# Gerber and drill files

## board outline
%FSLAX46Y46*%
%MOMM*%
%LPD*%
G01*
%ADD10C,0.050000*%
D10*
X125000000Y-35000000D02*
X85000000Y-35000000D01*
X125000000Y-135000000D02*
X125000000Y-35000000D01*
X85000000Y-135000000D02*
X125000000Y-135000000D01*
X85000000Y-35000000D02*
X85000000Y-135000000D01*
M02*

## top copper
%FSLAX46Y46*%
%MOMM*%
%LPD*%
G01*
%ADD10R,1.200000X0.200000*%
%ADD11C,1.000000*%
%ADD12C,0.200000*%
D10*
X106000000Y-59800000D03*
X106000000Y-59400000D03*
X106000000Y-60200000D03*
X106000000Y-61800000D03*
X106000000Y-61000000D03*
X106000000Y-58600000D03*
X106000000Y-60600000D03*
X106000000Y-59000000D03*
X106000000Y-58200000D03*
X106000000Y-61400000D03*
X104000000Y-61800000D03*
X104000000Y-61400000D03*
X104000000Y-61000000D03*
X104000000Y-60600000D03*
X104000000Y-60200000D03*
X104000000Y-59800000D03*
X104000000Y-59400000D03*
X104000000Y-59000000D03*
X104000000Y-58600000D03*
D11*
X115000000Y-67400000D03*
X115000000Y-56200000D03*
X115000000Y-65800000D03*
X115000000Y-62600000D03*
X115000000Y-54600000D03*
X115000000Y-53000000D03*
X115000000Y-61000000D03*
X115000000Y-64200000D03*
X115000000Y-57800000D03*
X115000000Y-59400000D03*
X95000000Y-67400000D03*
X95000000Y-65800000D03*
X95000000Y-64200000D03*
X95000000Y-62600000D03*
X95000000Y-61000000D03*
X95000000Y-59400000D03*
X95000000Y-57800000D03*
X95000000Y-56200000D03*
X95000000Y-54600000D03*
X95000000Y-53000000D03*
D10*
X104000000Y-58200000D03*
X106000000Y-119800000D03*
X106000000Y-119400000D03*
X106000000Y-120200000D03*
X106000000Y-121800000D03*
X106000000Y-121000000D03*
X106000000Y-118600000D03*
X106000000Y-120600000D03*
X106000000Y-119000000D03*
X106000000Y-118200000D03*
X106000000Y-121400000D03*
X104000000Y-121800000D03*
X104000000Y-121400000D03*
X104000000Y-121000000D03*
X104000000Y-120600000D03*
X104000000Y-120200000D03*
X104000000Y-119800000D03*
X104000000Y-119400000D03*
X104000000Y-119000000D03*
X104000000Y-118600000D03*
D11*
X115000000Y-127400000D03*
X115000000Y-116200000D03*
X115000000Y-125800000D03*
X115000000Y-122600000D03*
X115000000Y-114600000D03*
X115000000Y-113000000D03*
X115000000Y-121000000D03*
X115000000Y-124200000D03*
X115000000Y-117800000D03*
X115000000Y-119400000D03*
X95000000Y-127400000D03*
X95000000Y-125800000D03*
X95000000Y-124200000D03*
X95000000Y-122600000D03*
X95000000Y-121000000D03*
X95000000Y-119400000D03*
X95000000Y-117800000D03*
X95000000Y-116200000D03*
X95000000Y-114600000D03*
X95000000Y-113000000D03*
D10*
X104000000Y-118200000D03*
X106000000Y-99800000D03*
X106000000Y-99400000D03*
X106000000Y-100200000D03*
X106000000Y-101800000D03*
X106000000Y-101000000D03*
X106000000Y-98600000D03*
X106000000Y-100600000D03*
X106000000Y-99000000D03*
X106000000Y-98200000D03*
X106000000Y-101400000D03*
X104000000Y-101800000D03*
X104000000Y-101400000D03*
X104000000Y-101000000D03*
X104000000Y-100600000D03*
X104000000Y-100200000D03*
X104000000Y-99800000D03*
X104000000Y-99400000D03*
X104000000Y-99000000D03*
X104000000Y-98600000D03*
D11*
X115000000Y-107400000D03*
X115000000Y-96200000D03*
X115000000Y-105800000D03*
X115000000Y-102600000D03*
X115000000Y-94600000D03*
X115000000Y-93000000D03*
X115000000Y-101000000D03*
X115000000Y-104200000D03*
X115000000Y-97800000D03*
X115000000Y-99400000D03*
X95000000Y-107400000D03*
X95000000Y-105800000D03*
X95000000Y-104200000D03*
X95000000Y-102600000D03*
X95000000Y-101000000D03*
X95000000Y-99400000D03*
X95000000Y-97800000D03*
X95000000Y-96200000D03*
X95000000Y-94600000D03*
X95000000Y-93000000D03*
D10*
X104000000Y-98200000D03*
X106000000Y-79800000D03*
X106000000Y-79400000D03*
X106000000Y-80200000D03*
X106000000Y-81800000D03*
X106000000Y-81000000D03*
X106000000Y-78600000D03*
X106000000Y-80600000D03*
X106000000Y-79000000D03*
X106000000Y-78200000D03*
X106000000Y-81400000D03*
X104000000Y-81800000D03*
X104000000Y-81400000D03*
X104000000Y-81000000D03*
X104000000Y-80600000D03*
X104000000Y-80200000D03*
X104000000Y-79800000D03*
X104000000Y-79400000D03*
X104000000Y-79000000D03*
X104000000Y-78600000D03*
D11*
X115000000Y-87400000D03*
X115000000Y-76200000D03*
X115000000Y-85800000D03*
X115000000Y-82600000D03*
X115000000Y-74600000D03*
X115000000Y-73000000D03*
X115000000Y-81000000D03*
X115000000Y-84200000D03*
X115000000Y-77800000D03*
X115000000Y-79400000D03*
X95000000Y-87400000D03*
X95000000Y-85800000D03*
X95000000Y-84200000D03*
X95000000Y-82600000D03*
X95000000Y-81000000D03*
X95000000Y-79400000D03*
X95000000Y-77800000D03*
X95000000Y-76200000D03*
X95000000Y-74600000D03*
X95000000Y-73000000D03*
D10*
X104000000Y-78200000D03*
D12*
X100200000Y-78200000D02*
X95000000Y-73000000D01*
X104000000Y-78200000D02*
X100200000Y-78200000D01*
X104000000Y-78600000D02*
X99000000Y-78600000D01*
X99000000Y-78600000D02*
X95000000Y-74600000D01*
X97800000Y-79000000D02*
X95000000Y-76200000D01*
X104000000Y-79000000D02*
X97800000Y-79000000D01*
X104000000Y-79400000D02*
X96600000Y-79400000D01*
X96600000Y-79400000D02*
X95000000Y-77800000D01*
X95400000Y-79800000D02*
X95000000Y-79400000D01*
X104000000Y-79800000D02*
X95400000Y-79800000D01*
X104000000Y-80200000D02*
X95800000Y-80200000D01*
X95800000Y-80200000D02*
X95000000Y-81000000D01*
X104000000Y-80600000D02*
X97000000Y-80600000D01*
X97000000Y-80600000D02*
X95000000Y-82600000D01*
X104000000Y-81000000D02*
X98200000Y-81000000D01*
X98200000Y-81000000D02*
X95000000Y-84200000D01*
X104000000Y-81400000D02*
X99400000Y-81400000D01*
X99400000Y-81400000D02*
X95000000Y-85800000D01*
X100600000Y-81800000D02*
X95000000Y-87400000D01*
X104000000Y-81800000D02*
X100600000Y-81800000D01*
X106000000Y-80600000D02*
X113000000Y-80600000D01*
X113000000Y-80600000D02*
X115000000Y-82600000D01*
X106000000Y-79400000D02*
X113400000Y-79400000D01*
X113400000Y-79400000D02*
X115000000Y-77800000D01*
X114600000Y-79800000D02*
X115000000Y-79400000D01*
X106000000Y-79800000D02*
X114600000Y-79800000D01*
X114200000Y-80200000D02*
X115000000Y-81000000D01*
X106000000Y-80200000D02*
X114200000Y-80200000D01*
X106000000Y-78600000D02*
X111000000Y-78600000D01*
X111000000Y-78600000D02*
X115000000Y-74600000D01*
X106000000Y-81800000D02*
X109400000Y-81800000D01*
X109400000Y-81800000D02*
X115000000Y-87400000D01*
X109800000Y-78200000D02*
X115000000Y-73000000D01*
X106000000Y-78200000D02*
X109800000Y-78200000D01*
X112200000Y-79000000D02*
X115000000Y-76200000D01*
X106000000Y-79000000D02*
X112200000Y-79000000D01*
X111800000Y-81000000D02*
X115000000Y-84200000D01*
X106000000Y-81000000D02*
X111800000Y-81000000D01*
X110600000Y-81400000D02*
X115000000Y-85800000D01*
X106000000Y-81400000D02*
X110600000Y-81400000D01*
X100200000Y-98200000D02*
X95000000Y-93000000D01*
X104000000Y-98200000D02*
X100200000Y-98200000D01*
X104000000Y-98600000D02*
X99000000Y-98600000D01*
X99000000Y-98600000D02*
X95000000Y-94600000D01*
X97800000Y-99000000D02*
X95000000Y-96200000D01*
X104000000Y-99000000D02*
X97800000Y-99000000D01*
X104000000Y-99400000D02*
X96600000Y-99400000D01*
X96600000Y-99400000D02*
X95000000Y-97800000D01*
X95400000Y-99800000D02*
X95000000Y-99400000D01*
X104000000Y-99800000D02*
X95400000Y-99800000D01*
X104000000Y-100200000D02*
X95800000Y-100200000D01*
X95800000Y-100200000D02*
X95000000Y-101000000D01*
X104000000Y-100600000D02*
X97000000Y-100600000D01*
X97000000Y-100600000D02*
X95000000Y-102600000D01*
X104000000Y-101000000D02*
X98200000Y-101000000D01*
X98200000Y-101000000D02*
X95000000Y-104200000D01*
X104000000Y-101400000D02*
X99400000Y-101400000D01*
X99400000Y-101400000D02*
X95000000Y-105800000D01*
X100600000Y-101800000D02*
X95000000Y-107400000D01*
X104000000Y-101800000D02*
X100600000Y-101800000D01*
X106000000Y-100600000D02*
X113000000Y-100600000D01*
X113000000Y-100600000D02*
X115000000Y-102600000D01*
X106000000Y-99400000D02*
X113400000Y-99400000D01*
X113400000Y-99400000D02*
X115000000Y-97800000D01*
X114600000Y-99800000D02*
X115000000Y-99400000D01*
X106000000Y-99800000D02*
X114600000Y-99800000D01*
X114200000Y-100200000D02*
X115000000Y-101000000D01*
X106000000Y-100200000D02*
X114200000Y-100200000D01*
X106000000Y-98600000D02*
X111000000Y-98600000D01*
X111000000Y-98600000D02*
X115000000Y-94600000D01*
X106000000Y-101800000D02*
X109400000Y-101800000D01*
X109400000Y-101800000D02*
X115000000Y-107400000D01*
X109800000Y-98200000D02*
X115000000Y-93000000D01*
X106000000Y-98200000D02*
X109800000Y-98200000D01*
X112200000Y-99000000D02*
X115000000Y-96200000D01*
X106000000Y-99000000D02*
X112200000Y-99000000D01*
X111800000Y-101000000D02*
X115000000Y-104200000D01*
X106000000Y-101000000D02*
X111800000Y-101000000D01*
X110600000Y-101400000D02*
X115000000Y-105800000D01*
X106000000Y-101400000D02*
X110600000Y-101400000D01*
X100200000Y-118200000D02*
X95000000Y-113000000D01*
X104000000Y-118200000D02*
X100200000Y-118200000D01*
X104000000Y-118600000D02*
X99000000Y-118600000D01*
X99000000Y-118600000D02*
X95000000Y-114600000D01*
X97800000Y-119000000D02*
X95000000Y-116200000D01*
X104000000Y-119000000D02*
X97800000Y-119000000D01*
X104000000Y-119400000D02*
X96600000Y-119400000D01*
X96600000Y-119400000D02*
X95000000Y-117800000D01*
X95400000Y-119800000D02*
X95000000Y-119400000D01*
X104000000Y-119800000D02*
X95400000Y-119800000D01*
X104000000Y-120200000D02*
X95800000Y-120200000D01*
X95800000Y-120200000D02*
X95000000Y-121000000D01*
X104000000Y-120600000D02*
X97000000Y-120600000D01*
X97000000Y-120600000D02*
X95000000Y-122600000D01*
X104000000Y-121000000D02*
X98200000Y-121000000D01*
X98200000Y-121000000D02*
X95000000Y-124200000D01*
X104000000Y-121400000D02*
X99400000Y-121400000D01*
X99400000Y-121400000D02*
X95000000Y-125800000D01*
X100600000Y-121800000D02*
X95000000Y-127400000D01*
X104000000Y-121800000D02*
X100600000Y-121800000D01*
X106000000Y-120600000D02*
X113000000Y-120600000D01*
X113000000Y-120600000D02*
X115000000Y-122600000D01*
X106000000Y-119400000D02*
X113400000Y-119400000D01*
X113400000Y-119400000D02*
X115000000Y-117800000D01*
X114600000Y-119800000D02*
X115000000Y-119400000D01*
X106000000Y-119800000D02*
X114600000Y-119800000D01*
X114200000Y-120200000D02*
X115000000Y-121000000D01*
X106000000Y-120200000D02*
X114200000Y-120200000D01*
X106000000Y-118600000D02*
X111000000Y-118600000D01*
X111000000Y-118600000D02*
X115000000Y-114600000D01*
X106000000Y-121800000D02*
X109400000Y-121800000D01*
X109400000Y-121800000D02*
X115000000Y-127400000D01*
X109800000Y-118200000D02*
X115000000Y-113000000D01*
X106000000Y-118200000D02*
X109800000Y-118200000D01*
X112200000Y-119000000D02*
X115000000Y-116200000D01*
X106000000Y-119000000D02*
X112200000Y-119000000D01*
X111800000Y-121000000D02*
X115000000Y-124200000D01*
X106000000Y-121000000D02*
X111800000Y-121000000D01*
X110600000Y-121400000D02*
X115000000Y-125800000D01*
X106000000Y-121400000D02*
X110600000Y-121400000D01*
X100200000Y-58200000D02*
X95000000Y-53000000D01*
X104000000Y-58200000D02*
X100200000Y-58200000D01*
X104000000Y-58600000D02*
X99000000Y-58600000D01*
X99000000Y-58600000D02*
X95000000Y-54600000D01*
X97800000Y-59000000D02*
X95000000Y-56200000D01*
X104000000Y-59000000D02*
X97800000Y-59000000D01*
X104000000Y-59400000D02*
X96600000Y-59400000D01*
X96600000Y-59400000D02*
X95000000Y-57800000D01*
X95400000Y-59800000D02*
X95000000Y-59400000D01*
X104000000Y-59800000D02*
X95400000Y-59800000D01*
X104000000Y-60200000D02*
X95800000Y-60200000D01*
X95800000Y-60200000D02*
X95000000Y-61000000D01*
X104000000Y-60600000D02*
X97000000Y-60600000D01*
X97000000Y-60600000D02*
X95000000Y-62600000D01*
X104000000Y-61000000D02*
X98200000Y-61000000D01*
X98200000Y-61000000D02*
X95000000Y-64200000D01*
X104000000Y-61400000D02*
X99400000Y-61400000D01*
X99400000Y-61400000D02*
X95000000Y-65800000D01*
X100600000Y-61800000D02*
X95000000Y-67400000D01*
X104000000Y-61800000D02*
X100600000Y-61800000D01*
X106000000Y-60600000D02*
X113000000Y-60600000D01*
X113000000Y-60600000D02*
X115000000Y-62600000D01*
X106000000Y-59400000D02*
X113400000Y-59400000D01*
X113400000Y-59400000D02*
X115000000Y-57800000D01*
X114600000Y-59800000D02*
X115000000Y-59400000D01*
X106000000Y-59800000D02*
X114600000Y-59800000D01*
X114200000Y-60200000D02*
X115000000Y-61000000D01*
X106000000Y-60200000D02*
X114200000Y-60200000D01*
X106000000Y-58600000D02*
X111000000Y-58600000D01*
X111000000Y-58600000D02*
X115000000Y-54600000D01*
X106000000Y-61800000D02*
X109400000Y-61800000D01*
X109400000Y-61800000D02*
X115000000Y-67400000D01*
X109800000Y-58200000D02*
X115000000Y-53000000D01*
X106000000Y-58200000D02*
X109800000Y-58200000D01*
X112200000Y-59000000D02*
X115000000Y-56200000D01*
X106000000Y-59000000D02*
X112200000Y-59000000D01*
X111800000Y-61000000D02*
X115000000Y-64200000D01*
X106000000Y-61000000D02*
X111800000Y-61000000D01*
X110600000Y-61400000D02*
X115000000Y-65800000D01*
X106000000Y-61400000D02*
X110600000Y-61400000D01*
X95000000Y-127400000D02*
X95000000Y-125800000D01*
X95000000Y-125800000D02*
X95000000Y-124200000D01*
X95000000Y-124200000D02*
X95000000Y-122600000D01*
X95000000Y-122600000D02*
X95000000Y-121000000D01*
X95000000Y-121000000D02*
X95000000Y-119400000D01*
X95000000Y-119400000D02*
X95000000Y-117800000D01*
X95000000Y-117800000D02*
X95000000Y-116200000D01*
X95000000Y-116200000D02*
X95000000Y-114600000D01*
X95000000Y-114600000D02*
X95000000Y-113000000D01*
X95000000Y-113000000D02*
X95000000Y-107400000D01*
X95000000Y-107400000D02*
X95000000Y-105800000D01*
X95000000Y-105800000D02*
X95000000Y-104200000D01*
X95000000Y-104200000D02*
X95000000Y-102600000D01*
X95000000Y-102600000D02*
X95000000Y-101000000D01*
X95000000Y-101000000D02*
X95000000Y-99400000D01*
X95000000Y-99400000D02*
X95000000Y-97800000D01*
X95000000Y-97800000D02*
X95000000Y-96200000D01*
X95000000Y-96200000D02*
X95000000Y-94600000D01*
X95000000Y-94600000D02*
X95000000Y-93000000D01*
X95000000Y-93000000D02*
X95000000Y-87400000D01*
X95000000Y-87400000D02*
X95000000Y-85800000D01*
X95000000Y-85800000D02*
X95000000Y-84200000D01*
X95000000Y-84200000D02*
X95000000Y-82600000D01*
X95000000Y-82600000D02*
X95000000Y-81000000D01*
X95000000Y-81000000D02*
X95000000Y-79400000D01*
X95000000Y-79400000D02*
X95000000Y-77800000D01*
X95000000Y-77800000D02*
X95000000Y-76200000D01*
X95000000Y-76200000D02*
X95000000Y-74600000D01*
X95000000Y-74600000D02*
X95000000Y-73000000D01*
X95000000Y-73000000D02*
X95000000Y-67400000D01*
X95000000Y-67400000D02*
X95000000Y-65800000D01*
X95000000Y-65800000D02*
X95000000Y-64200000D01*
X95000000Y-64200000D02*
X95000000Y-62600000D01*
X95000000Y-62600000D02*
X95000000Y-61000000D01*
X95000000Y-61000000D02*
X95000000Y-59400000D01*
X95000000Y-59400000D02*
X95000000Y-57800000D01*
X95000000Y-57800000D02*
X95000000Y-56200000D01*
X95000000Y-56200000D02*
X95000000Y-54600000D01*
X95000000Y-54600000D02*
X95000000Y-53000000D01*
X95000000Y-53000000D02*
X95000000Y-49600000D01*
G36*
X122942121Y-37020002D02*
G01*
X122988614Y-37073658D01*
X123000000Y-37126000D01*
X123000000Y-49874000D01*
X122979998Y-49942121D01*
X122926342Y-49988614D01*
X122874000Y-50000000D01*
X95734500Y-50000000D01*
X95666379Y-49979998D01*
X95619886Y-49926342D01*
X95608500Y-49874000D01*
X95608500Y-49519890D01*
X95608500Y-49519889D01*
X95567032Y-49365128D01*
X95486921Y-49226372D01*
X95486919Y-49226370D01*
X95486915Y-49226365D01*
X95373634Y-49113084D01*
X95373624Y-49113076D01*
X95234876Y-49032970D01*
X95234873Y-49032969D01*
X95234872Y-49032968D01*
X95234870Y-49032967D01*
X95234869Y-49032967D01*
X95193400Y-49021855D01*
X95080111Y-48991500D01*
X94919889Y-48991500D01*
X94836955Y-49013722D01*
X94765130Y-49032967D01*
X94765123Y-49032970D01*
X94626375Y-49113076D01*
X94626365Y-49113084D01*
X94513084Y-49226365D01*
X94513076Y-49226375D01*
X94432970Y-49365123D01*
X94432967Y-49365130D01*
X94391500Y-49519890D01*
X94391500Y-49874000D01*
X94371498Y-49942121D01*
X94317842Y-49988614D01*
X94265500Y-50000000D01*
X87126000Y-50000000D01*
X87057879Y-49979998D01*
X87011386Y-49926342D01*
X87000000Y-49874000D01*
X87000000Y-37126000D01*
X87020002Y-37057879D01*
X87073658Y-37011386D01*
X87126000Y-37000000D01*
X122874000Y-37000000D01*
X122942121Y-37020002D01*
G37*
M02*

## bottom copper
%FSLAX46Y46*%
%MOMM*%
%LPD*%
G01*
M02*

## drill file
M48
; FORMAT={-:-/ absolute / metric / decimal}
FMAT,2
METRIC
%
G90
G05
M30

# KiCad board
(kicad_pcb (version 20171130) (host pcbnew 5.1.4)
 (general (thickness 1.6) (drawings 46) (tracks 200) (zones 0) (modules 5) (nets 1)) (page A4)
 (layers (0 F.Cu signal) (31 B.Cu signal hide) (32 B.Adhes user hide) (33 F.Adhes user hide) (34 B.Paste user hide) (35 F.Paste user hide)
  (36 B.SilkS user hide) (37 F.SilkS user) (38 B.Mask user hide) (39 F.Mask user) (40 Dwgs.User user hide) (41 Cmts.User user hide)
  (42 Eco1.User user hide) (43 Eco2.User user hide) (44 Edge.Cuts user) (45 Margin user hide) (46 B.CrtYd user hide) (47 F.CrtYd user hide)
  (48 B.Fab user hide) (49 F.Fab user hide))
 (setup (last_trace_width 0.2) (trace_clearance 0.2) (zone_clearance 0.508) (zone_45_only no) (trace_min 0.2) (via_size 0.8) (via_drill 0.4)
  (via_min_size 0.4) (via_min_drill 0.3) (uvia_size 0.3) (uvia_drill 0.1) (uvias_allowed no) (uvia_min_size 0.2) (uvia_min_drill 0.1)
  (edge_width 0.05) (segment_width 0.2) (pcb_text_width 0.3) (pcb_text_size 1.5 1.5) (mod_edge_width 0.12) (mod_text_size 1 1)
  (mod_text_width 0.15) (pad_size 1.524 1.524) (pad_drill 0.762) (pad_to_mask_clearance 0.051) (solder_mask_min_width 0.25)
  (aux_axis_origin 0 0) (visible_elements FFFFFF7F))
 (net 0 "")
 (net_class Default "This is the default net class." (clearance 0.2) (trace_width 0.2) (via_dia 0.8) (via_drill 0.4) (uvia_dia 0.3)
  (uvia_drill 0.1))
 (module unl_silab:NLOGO (layer F.Cu) (at 87.6 132.2)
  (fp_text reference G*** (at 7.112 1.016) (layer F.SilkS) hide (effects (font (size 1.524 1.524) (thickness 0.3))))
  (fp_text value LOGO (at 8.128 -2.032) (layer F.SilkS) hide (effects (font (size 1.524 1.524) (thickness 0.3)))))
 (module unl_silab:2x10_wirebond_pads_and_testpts (layer F.Cu) (at 105 60)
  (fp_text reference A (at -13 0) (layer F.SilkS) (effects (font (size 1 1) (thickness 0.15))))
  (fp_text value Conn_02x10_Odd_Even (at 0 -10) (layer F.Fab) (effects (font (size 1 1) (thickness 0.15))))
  (pad 15 smd rect (at 1 -0.2) (size 1.2 0.2) (layers F.Cu F.Paste F.Mask))
  (pad 14 smd rect (at 1 -0.6) (size 1.2 0.2) (layers F.Cu F.Paste F.Mask))
  (pad 16 smd rect (at 1 0.2) (size 1.2 0.2) (layers F.Cu F.Paste F.Mask))
  (pad 20 smd rect (at 1 1.8) (size 1.2 0.2) (layers F.Cu F.Paste F.Mask))
  (pad 18 smd rect (at 1 1) (size 1.2 0.2) (layers F.Cu F.Paste F.Mask))
  (pad 12 smd rect (at 1 -1.4) (size 1.2 0.2) (layers F.Cu F.Paste F.Mask))
  (pad 17 smd rect (at 1 0.6) (size 1.2 0.2) (layers F.Cu F.Paste F.Mask))
  (pad 13 smd rect (at 1 -1) (size 1.2 0.2) (layers F.Cu F.Paste F.Mask))
  (pad 11 smd rect (at 1 -1.8) (size 1.2 0.2) (layers F.Cu F.Paste F.Mask))
  (pad 19 smd rect (at 1 1.4) (size 1.2 0.2) (layers F.Cu F.Paste F.Mask))
  (pad 10 smd rect (at -1 1.8) (size 1.2 0.2) (layers F.Cu F.Paste F.Mask))
  (pad 9 smd rect (at -1 1.4) (size 1.2 0.2) (layers F.Cu F.Paste F.Mask))
  (pad 8 smd rect (at -1 1) (size 1.2 0.2) (layers F.Cu F.Paste F.Mask))
  (pad 7 smd rect (at -1 0.6) (size 1.2 0.2) (layers F.Cu F.Paste F.Mask))
  (pad 6 smd rect (at -1 0.2) (size 1.2 0.2) (layers F.Cu F.Paste F.Mask))
  (pad 5 smd rect (at -1 -0.2) (size 1.2 0.2) (layers F.Cu F.Paste F.Mask))
  (pad 4 smd rect (at -1 -0.6) (size 1.2 0.2) (layers F.Cu F.Paste F.Mask))
  (pad 3 smd rect (at -1 -1) (size 1.2 0.2) (layers F.Cu F.Paste F.Mask))
  (pad 2 smd rect (at -1 -1.4) (size 1.2 0.2) (layers F.Cu F.Paste F.Mask))
  (pad 20 smd circle (at 10 7.4) (size 1 1) (layers F.Cu F.Paste F.Mask))
  (pad 13 smd circle (at 10 -3.8) (size 1 1) (layers F.Cu F.Paste F.Mask))
  (pad 19 smd circle (at 10 5.8) (size 1 1) (layers F.Cu F.Paste F.Mask))
  (pad 17 smd circle (at 10 2.6) (size 1 1) (layers F.Cu F.Paste F.Mask))
  (pad 12 smd circle (at 10 -5.4) (size 1 1) (layers F.Cu F.Paste F.Mask))
  (pad 11 smd circle (at 10 -7) (size 1 1) (layers F.Cu F.Paste F.Mask))
  (pad 16 smd circle (at 10 1) (size 1 1) (layers F.Cu F.Paste F.Mask))
  (pad 18 smd circle (at 10 4.2) (size 1 1) (layers F.Cu F.Paste F.Mask))
  (pad 14 smd circle (at 10 -2.2) (size 1 1) (layers F.Cu F.Paste F.Mask))
  (pad 15 smd circle (at 10 -0.6) (size 1 1) (layers F.Cu F.Paste F.Mask))
  (pad 10 smd circle (at -10 7.4) (size 1 1) (layers F.Cu F.Paste F.Mask))
  (pad 9 smd circle (at -10 5.8) (size 1 1) (layers F.Cu F.Paste F.Mask))
  (pad 8 smd circle (at -10 4.2) (size 1 1) (layers F.Cu F.Paste F.Mask))
  (pad 7 smd circle (at -10 2.6) (size 1 1) (layers F.Cu F.Paste F.Mask))
  (pad 6 smd circle (at -10 1) (size 1 1) (layers F.Cu F.Paste F.Mask))
  (pad 5 smd circle (at -10 -0.6) (size 1 1) (layers F.Cu F.Paste F.Mask))
  (pad 4 smd circle (at -10 -2.2) (size 1 1) (layers F.Cu F.Paste F.Mask))
  (pad 3 smd circle (at -10 -3.8) (size 1 1) (layers F.Cu F.Paste F.Mask))
  (pad 2 smd circle (at -10 -5.4) (size 1 1) (layers F.Cu F.Paste F.Mask))
  (pad 1 smd circle (at -10 -7) (size 1 1) (layers F.Cu F.Paste F.Mask))
  (pad 1 smd rect (at -1 -1.8) (size 1.2 0.2) (layers F.Cu F.Paste F.Mask)))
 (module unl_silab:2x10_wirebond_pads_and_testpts (layer F.Cu) (at 105 120)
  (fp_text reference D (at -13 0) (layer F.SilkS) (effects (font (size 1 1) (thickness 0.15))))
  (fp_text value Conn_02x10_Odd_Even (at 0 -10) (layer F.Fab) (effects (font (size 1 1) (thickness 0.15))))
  (pad 15 smd rect (at 1 -0.2) (size 1.2 0.2) (layers F.Cu F.Paste F.Mask))
  (pad 14 smd rect (at 1 -0.6) (size 1.2 0.2) (layers F.Cu F.Paste F.Mask))
  (pad 16 smd rect (at 1 0.2) (size 1.2 0.2) (layers F.Cu F.Paste F.Mask))
  (pad 20 smd rect (at 1 1.8) (size 1.2 0.2) (layers F.Cu F.Paste F.Mask))
  (pad 18 smd rect (at 1 1) (size 1.2 0.2) (layers F.Cu F.Paste F.Mask))
  (pad 12 smd rect (at 1 -1.4) (size 1.2 0.2) (layers F.Cu F.Paste F.Mask))
  (pad 17 smd rect (at 1 0.6) (size 1.2 0.2) (layers F.Cu F.Paste F.Mask))
  (pad 13 smd rect (at 1 -1) (size 1.2 0.2) (layers F.Cu F.Paste F.Mask))
  (pad 11 smd rect (at 1 -1.8) (size 1.2 0.2) (layers F.Cu F.Paste F.Mask))
  (pad 19 smd rect (at 1 1.4) (size 1.2 0.2) (layers F.Cu F.Paste F.Mask))
  (pad 10 smd rect (at -1 1.8) (size 1.2 0.2) (layers F.Cu F.Paste F.Mask))
  (pad 9 smd rect (at -1 1.4) (size 1.2 0.2) (layers F.Cu F.Paste F.Mask))
  (pad 8 smd rect (at -1 1) (size 1.2 0.2) (layers F.Cu F.Paste F.Mask))
  (pad 7 smd rect (at -1 0.6) (size 1.2 0.2) (layers F.Cu F.Paste F.Mask))
  (pad 6 smd rect (at -1 0.2) (size 1.2 0.2) (layers F.Cu F.Paste F.Mask))
  (pad 5 smd rect (at -1 -0.2) (size 1.2 0.2) (layers F.Cu F.Paste F.Mask))
  (pad 4 smd rect (at -1 -0.6) (size 1.2 0.2) (layers F.Cu F.Paste F.Mask))
  (pad 3 smd rect (at -1 -1) (size 1.2 0.2) (layers F.Cu F.Paste F.Mask))
  (pad 2 smd rect (at -1 -1.4) (size 1.2 0.2) (layers F.Cu F.Paste F.Mask))
  (pad 20 smd circle (at 10 7.4) (size 1 1) (layers F.Cu F.Paste F.Mask))
  (pad 13 smd circle (at 10 -3.8) (size 1 1) (layers F.Cu F.Paste F.Mask))
  (pad 19 smd circle (at 10 5.8) (size 1 1) (layers F.Cu F.Paste F.Mask))
  (pad 17 smd circle (at 10 2.6) (size 1 1) (layers F.Cu F.Paste F.Mask))
  (pad 12 smd circle (at 10 -5.4) (size 1 1) (layers F.Cu F.Paste F.Mask))
  (pad 11 smd circle (at 10 -7) (size 1 1) (layers F.Cu F.Paste F.Mask))
  (pad 16 smd circle (at 10 1) (size 1 1) (layers F.Cu F.Paste F.Mask))
  (pad 18 smd circle (at 10 4.2) (size 1 1) (layers F.Cu F.Paste F.Mask))
  (pad 14 smd circle (at 10 -2.2) (size 1 1) (layers F.Cu F.Paste F.Mask))
  (pad 15 smd circle (at 10 -0.6) (size 1 1) (layers F.Cu F.Paste F.Mask))
  (pad 10 smd circle (at -10 7.4) (size 1 1) (layers F.Cu F.Paste F.Mask))
  (pad 9 smd circle (at -10 5.8) (size 1 1) (layers F.Cu F.Paste F.Mask))
  (pad 8 smd circle (at -10 4.2) (size 1 1) (layers F.Cu F.Paste F.Mask))
  (pad 7 smd circle (at -10 2.6) (size 1 1) (layers F.Cu F.Paste F.Mask))
  (pad 6 smd circle (at -10 1) (size 1 1) (layers F.Cu F.Paste F.Mask))
  (pad 5 smd circle (at -10 -0.6) (size 1 1) (layers F.Cu F.Paste F.Mask))
  (pad 4 smd circle (at -10 -2.2) (size 1 1) (layers F.Cu F.Paste F.Mask))
  (pad 3 smd circle (at -10 -3.8) (size 1 1) (layers F.Cu F.Paste F.Mask))
  (pad 2 smd circle (at -10 -5.4) (size 1 1) (layers F.Cu F.Paste F.Mask))
  (pad 1 smd circle (at -10 -7) (size 1 1) (layers F.Cu F.Paste F.Mask))
  (pad 1 smd rect (at -1 -1.8) (size 1.2 0.2) (layers F.Cu F.Paste F.Mask)))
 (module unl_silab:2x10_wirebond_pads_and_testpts (layer F.Cu) (at 105 100)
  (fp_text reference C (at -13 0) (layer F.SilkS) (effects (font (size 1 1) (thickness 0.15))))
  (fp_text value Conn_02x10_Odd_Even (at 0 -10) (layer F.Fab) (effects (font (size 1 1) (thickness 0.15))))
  (pad 15 smd rect (at 1 -0.2) (size 1.2 0.2) (layers F.Cu F.Paste F.Mask))
  (pad 14 smd rect (at 1 -0.6) (size 1.2 0.2) (layers F.Cu F.Paste F.Mask))
  (pad 16 smd rect (at 1 0.2) (size 1.2 0.2) (layers F.Cu F.Paste F.Mask))
  (pad 20 smd rect (at 1 1.8) (size 1.2 0.2) (layers F.Cu F.Paste F.Mask))
  (pad 18 smd rect (at 1 1) (size 1.2 0.2) (layers F.Cu F.Paste F.Mask))
  (pad 12 smd rect (at 1 -1.4) (size 1.2 0.2) (layers F.Cu F.Paste F.Mask))
  (pad 17 smd rect (at 1 0.6) (size 1.2 0.2) (layers F.Cu F.Paste F.Mask))
  (pad 13 smd rect (at 1 -1) (size 1.2 0.2) (layers F.Cu F.Paste F.Mask))
  (pad 11 smd rect (at 1 -1.8) (size 1.2 0.2) (layers F.Cu F.Paste F.Mask))
  (pad 19 smd rect (at 1 1.4) (size 1.2 0.2) (layers F.Cu F.Paste F.Mask))
  (pad 10 smd rect (at -1 1.8) (size 1.2 0.2) (layers F.Cu F.Paste F.Mask))
  (pad 9 smd rect (at -1 1.4) (size 1.2 0.2) (layers F.Cu F.Paste F.Mask))
  (pad 8 smd rect (at -1 1) (size 1.2 0.2) (layers F.Cu F.Paste F.Mask))
  (pad 7 smd rect (at -1 0.6) (size 1.2 0.2) (layers F.Cu F.Paste F.Mask))
  (pad 6 smd rect (at -1 0.2) (size 1.2 0.2) (layers F.Cu F.Paste F.Mask))
  (pad 5 smd rect (at -1 -0.2) (size 1.2 0.2) (layers F.Cu F.Paste F.Mask))
  (pad 4 smd rect (at -1 -0.6) (size 1.2 0.2) (layers F.Cu F.Paste F.Mask))
  (pad 3 smd rect (at -1 -1) (size 1.2 0.2) (layers F.Cu F.Paste F.Mask))
  (pad 2 smd rect (at -1 -1.4) (size 1.2 0.2) (layers F.Cu F.Paste F.Mask))
  (pad 20 smd circle (at 10 7.4) (size 1 1) (layers F.Cu F.Paste F.Mask))
  (pad 13 smd circle (at 10 -3.8) (size 1 1) (layers F.Cu F.Paste F.Mask))
  (pad 19 smd circle (at 10 5.8) (size 1 1) (layers F.Cu F.Paste F.Mask))
  (pad 17 smd circle (at 10 2.6) (size 1 1) (layers F.Cu F.Paste F.Mask))
  (pad 12 smd circle (at 10 -5.4) (size 1 1) (layers F.Cu F.Paste F.Mask))
  (pad 11 smd circle (at 10 -7) (size 1 1) (layers F.Cu F.Paste F.Mask))
  (pad 16 smd circle (at 10 1) (size 1 1) (layers F.Cu F.Paste F.Mask))
  (pad 18 smd circle (at 10 4.2) (size 1 1) (layers F.Cu F.Paste F.Mask))
  (pad 14 smd circle (at 10 -2.2) (size 1 1) (layers F.Cu F.Paste F.Mask))
  (pad 15 smd circle (at 10 -0.6) (size 1 1) (layers F.Cu F.Paste F.Mask))
  (pad 10 smd circle (at -10 7.4) (size 1 1) (layers F.Cu F.Paste F.Mask))
  (pad 9 smd circle (at -10 5.8) (size 1 1) (layers F.Cu F.Paste F.Mask))
  (pad 8 smd circle (at -10 4.2) (size 1 1) (layers F.Cu F.Paste F.Mask))
  (pad 7 smd circle (at -10 2.6) (size 1 1) (layers F.Cu F.Paste F.Mask))
  (pad 6 smd circle (at -10 1) (size 1 1) (layers F.Cu F.Paste F.Mask))
  (pad 5 smd circle (at -10 -0.6) (size 1 1) (layers F.Cu F.Paste F.Mask))
  (pad 4 smd circle (at -10 -2.2) (size 1 1) (layers F.Cu F.Paste F.Mask))
  (pad 3 smd circle (at -10 -3.8) (size 1 1) (layers F.Cu F.Paste F.Mask))
  (pad 2 smd circle (at -10 -5.4) (size 1 1) (layers F.Cu F.Paste F.Mask))
  (pad 1 smd circle (at -10 -7) (size 1 1) (layers F.Cu F.Paste F.Mask))
  (pad 1 smd rect (at -1 -1.8) (size 1.2 0.2) (layers F.Cu F.Paste F.Mask)))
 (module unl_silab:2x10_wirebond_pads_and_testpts (layer F.Cu) (at 105 80)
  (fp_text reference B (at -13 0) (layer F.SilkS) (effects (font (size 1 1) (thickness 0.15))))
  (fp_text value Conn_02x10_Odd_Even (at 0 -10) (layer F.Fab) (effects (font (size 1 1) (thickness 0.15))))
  (pad 15 smd rect (at 1 -0.2) (size 1.2 0.2) (layers F.Cu F.Paste F.Mask))
  (pad 14 smd rect (at 1 -0.6) (size 1.2 0.2) (layers F.Cu F.Paste F.Mask))
  (pad 16 smd rect (at 1 0.2) (size 1.2 0.2) (layers F.Cu F.Paste F.Mask))
  (pad 20 smd rect (at 1 1.8) (size 1.2 0.2) (layers F.Cu F.Paste F.Mask))
  (pad 18 smd rect (at 1 1) (size 1.2 0.2) (layers F.Cu F.Paste F.Mask))
  (pad 12 smd rect (at 1 -1.4) (size 1.2 0.2) (layers F.Cu F.Paste F.Mask))
  (pad 17 smd rect (at 1 0.6) (size 1.2 0.2) (layers F.Cu F.Paste F.Mask))
  (pad 13 smd rect (at 1 -1) (size 1.2 0.2) (layers F.Cu F.Paste F.Mask))
  (pad 11 smd rect (at 1 -1.8) (size 1.2 0.2) (layers F.Cu F.Paste F.Mask))
  (pad 19 smd rect (at 1 1.4) (size 1.2 0.2) (layers F.Cu F.Paste F.Mask))
  (pad 10 smd rect (at -1 1.8) (size 1.2 0.2) (layers F.Cu F.Paste F.Mask))
  (pad 9 smd rect (at -1 1.4) (size 1.2 0.2) (layers F.Cu F.Paste F.Mask))
  (pad 8 smd rect (at -1 1) (size 1.2 0.2) (layers F.Cu F.Paste F.Mask))
  (pad 7 smd rect (at -1 0.6) (size 1.2 0.2) (layers F.Cu F.Paste F.Mask))
  (pad 6 smd rect (at -1 0.2) (size 1.2 0.2) (layers F.Cu F.Paste F.Mask))
  (pad 5 smd rect (at -1 -0.2) (size 1.2 0.2) (layers F.Cu F.Paste F.Mask))
  (pad 4 smd rect (at -1 -0.6) (size 1.2 0.2) (layers F.Cu F.Paste F.Mask))
  (pad 3 smd rect (at -1 -1) (size 1.2 0.2) (layers F.Cu F.Paste F.Mask))
  (pad 2 smd rect (at -1 -1.4) (size 1.2 0.2) (layers F.Cu F.Paste F.Mask))
  (pad 20 smd circle (at 10 7.4) (size 1 1) (layers F.Cu F.Paste F.Mask))
  (pad 13 smd circle (at 10 -3.8) (size 1 1) (layers F.Cu F.Paste F.Mask))
  (pad 19 smd circle (at 10 5.8) (size 1 1) (layers F.Cu F.Paste F.Mask))
  (pad 17 smd circle (at 10 2.6) (size 1 1) (layers F.Cu F.Paste F.Mask))
  (pad 12 smd circle (at 10 -5.4) (size 1 1) (layers F.Cu F.Paste F.Mask))
  (pad 11 smd circle (at 10 -7) (size 1 1) (layers F.Cu F.Paste F.Mask))
  (pad 16 smd circle (at 10 1) (size 1 1) (layers F.Cu F.Paste F.Mask))
  (pad 18 smd circle (at 10 4.2) (size 1 1) (layers F.Cu F.Paste F.Mask))
  (pad 14 smd circle (at 10 -2.2) (size 1 1) (layers F.Cu F.Paste F.Mask))
  (pad 15 smd circle (at 10 -0.6) (size 1 1) (layers F.Cu F.Paste F.Mask))
  (pad 10 smd circle (at -10 7.4) (size 1 1) (layers F.Cu F.Paste F.Mask))
  (pad 9 smd circle (at -10 5.8) (size 1 1) (layers F.Cu F.Paste F.Mask))
  (pad 8 smd circle (at -10 4.2) (size 1 1) (layers F.Cu F.Paste F.Mask))
  (pad 7 smd circle (at -10 2.6) (size 1 1) (layers F.Cu F.Paste F.Mask))
  (pad 6 smd circle (at -10 1) (size 1 1) (layers F.Cu F.Paste F.Mask))
  (pad 5 smd circle (at -10 -0.6) (size 1 1) (layers F.Cu F.Paste F.Mask))
  (pad 4 smd circle (at -10 -2.2) (size 1 1) (layers F.Cu F.Paste F.Mask))
  (pad 3 smd circle (at -10 -3.8) (size 1 1) (layers F.Cu F.Paste F.Mask))
  (pad 2 smd circle (at -10 -5.4) (size 1 1) (layers F.Cu F.Paste F.Mask))
  (pad 1 smd circle (at -10 -7) (size 1 1) (layers F.Cu F.Paste F.Mask))
  (pad 1 smd rect (at -1 -1.8) (size 1.2 0.2) (layers F.Cu F.Paste F.Mask)))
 (gr_line (start 125 35) (end 85 35) (layer Edge.Cuts) (width 0.05))
 (gr_line (start 125 135) (end 125 35) (layer Edge.Cuts) (width 0.05))
 (gr_line (start 85 135) (end 125 135) (layer Edge.Cuts) (width 0.05))
 (gr_line (start 85 35) (end 85 135) (layer Edge.Cuts) (width 0.05))
 (segment (start 100.2 78.2) (end 95 73) (width 0.2) (layer F.Cu) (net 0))
 (segment (start 104 78.2) (end 100.2 78.2) (width 0.2) (layer F.Cu) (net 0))
 (segment (start 104 78.6) (end 99 78.6) (width 0.2) (layer F.Cu) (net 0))
 (segment (start 99 78.6) (end 95 74.6) (width 0.2) (layer F.Cu) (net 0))
 (segment (start 97.8 79) (end 95 76.2) (width 0.2) (layer F.Cu) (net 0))
 (segment (start 104 79) (end 97.8 79) (width 0.2) (layer F.Cu) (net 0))
 (segment (start 104 79.4) (end 96.6 79.4) (width 0.2) (layer F.Cu) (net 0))
 (segment (start 96.6 79.4) (end 95 77.8) (width 0.2) (layer F.Cu) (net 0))
 (segment (start 95.4 79.8) (end 95 79.4) (width 0.2) (layer F.Cu) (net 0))
 (segment (start 104 79.8) (end 95.4 79.8) (width 0.2) (layer F.Cu) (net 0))
 (segment (start 104 80.2) (end 95.8 80.2) (width 0.2) (layer F.Cu) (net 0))
 (segment (start 95.8 80.2) (end 95 81) (width 0.2) (layer F.Cu) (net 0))
 (segment (start 104 80.6) (end 97 80.6) (width 0.2) (layer F.Cu) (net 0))
 (segment (start 97 80.6) (end 95 82.6) (width 0.2) (layer F.Cu) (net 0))
 (segment (start 104 81) (end 98.2 81) (width 0.2) (layer F.Cu) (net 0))
 (segment (start 98.2 81) (end 95 84.2) (width 0.2) (layer F.Cu) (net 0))
 (segment (start 104 81.4) (end 99.4 81.4) (width 0.2) (layer F.Cu) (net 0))
 (segment (start 99.4 81.4) (end 95 85.8) (width 0.2) (layer F.Cu) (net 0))
 (segment (start 100.6 81.8) (end 95 87.4) (width 0.2) (layer F.Cu) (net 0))
 (segment (start 104 81.8) (end 100.6 81.8) (width 0.2) (layer F.Cu) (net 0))
 (segment (start 106 80.6) (end 113 80.6) (width 0.2) (layer F.Cu) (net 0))
 (segment (start 113 80.6) (end 115 82.6) (width 0.2) (layer F.Cu) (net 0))
 (segment (start 106 79.4) (end 113.4 79.4) (width 0.2) (layer F.Cu) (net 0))
 (segment (start 113.4 79.4) (end 115 77.8) (width 0.2) (layer F.Cu) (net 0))
 (segment (start 114.6 79.8) (end 115 79.4) (width 0.2) (layer F.Cu) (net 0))
 (segment (start 106 79.8) (end 114.6 79.8) (width 0.2) (layer F.Cu) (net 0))
 (segment (start 114.2 80.2) (end 115 81) (width 0.2) (layer F.Cu) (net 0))
 (segment (start 106 80.2) (end 114.2 80.2) (width 0.2) (layer F.Cu) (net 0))
 (segment (start 106 78.6) (end 111 78.6) (width 0.2) (layer F.Cu) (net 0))
 (segment (start 111 78.6) (end 115 74.6) (width 0.2) (layer F.Cu) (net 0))
 (segment (start 106 81.8) (end 109.4 81.8) (width 0.2) (layer F.Cu) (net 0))
 (segment (start 109.4 81.8) (end 115 87.4) (width 0.2) (layer F.Cu) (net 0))
 (segment (start 109.8 78.2) (end 115 73) (width 0.2) (layer F.Cu) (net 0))
 (segment (start 106 78.2) (end 109.8 78.2) (width 0.2) (layer F.Cu) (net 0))
 (segment (start 112.2 79) (end 115 76.2) (width 0.2) (layer F.Cu) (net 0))
 (segment (start 106 79) (end 112.2 79) (width 0.2) (layer F.Cu) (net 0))
 (segment (start 111.8 81) (end 115 84.2) (width 0.2) (layer F.Cu) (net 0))
 (segment (start 106 81) (end 111.8 81) (width 0.2) (layer F.Cu) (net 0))
 (segment (start 110.6 81.4) (end 115 85.8) (width 0.2) (layer F.Cu) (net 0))
 (segment (start 106 81.4) (end 110.6 81.4) (width 0.2) (layer F.Cu) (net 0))
 (segment (start 100.2 98.2) (end 95 93) (width 0.2) (layer F.Cu) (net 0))
 (segment (start 104 98.2) (end 100.2 98.2) (width 0.2) (layer F.Cu) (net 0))
 (segment (start 104 98.6) (end 99 98.6) (width 0.2) (layer F.Cu) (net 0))
 (segment (start 99 98.6) (end 95 94.6) (width 0.2) (layer F.Cu) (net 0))
 (segment (start 97.8 99) (end 95 96.2) (width 0.2) (layer F.Cu) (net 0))
 (segment (start 104 99) (end 97.8 99) (width 0.2) (layer F.Cu) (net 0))
 (segment (start 104 99.4) (end 96.6 99.4) (width 0.2) (layer F.Cu) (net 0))
 (segment (start 96.6 99.4) (end 95 97.8) (width 0.2) (layer F.Cu) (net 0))
 (segment (start 95.4 99.8) (end 95 99.4) (width 0.2) (layer F.Cu) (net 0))
 (segment (start 104 99.8) (end 95.4 99.8) (width 0.2) (layer F.Cu) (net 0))
 (segment (start 104 100.2) (end 95.8 100.2) (width 0.2) (layer F.Cu) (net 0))
 (segment (start 95.8 100.2) (end 95 101) (width 0.2) (layer F.Cu) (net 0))
 (segment (start 104 100.6) (end 97 100.6) (width 0.2) (layer F.Cu) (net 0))
 (segment (start 97 100.6) (end 95 102.6) (width 0.2) (layer F.Cu) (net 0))
 (segment (start 104 101) (end 98.2 101) (width 0.2) (layer F.Cu) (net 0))
 (segment (start 98.2 101) (end 95 104.2) (width 0.2) (layer F.Cu) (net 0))
 (segment (start 104 101.4) (end 99.4 101.4) (width 0.2) (layer F.Cu) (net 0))
 (segment (start 99.4 101.4) (end 95 105.8) (width 0.2) (layer F.Cu) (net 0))
 (segment (start 100.6 101.8) (end 95 107.4) (width 0.2) (layer F.Cu) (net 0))
 (segment (start 104 101.8) (end 100.6 101.8) (width 0.2) (layer F.Cu) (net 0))
 (segment (start 106 100.6) (end 113 100.6) (width 0.2) (layer F.Cu) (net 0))
 (segment (start 113 100.6) (end 115 102.6) (width 0.2) (layer F.Cu) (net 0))
 (segment (start 106 99.4) (end 113.4 99.4) (width 0.2) (layer F.Cu) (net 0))
 (segment (start 113.4 99.4) (end 115 97.8) (width 0.2) (layer F.Cu) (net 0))
 (segment (start 114.6 99.8) (end 115 99.4) (width 0.2) (layer F.Cu) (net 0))
 (segment (start 106 99.8) (end 114.6 99.8) (width 0.2) (layer F.Cu) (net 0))
 (segment (start 114.2 100.2) (end 115 101) (width 0.2) (layer F.Cu) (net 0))
 (segment (start 106 100.2) (end 114.2 100.2) (width 0.2) (layer F.Cu) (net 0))
 (segment (start 106 98.6) (end 111 98.6) (width 0.2) (layer F.Cu) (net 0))
 (segment (start 111 98.6) (end 115 94.6) (width 0.2) (layer F.Cu) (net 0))
 (segment (start 106 101.8) (end 109.4 101.8) (width 0.2) (layer F.Cu) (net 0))
 (segment (start 109.4 101.8) (end 115 107.4) (width 0.2) (layer F.Cu) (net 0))
 (segment (start 109.8 98.2) (end 115 93) (width 0.2) (layer F.Cu) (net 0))
 (segment (start 106 98.2) (end 109.8 98.2) (width 0.2) (layer F.Cu) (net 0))
 (segment (start 112.2 99) (end 115 96.2) (width 0.2) (layer F.Cu) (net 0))
 (segment (start 106 99) (end 112.2 99) (width 0.2) (layer F.Cu) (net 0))
 (segment (start 111.8 101) (end 115 104.2) (width 0.2) (layer F.Cu) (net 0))
 (segment (start 106 101) (end 111.8 101) (width 0.2) (layer F.Cu) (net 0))
 (segment (start 110.6 101.4) (end 115 105.8) (width 0.2) (layer F.Cu) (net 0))
 (segment (start 106 101.4) (end 110.6 101.4) (width 0.2) (layer F.Cu) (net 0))
 (segment (start 100.2 118.2) (end 95 113) (width 0.2) (layer F.Cu) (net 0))
 (segment (start 104 118.2) (end 100.2 118.2) (width 0.2) (layer F.Cu) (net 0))
 (segment (start 104 118.6) (end 99 118.6) (width 0.2) (layer F.Cu) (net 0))
 (segment (start 99 118.6) (end 95 114.6) (width 0.2) (layer F.Cu) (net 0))
 (segment (start 97.8 119) (end 95 116.2) (width 0.2) (layer F.Cu) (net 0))
 (segment (start 104 119) (end 97.8 119) (width 0.2) (layer F.Cu) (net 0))
 (segment (start 104 119.4) (end 96.6 119.4) (width 0.2) (layer F.Cu) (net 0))
 (segment (start 96.6 119.4) (end 95 117.8) (width 0.2) (layer F.Cu) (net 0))
 (segment (start 95.4 119.8) (end 95 119.4) (width 0.2) (layer F.Cu) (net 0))
 (segment (start 104 119.8) (end 95.4 119.8) (width 0.2) (layer F.Cu) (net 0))
 (segment (start 104 120.2) (end 95.8 120.2) (width 0.2) (layer F.Cu) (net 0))
 (segment (start 95.8 120.2) (end 95 121) (width 0.2) (layer F.Cu) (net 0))
 (segment (start 104 120.6) (end 97 120.6) (width 0.2) (layer F.Cu) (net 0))
 (segment (start 97 120.6) (end 95 122.6) (width 0.2) (layer F.Cu) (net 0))
 (segment (start 104 121) (end 98.2 121) (width 0.2) (layer F.Cu) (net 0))
 (segment (start 98.2 121) (end 95 124.2) (width 0.2) (layer F.Cu) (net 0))
 (segment (start 104 121.4) (end 99.4 121.4) (width 0.2) (layer F.Cu) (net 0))
 (segment (start 99.4 121.4) (end 95 125.8) (width 0.2) (layer F.Cu) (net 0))
 (segment (start 100.6 121.8) (end 95 127.4) (width 0.2) (layer F.Cu) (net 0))
 (segment (start 104 121.8) (end 100.6 121.8) (width 0.2) (layer F.Cu) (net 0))
 (segment (start 106 120.6) (end 113 120.6) (width 0.2) (layer F.Cu) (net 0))
 (segment (start 113 120.6) (end 115 122.6) (width 0.2) (layer F.Cu) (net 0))
 (segment (start 106 119.4) (end 113.4 119.4) (width 0.2) (layer F.Cu) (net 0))
 (segment (start 113.4 119.4) (end 115 117.8) (width 0.2) (layer F.Cu) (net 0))
 (segment (start 114.6 119.8) (end 115 119.4) (width 0.2) (layer F.Cu) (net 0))
 (segment (start 106 119.8) (end 114.6 119.8) (width 0.2) (layer F.Cu) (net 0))
 (segment (start 114.2 120.2) (end 115 121) (width 0.2) (layer F.Cu) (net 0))
 (segment (start 106 120.2) (end 114.2 120.2) (width 0.2) (layer F.Cu) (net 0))
 (segment (start 106 118.6) (end 111 118.6) (width 0.2) (layer F.Cu) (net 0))
 (segment (start 111 118.6) (end 115 114.6) (width 0.2) (layer F.Cu) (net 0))
 (segment (start 106 121.8) (end 109.4 121.8) (width 0.2) (layer F.Cu) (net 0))
 (segment (start 109.4 121.8) (end 115 127.4) (width 0.2) (layer F.Cu) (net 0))
 (segment (start 109.8 118.2) (end 115 113) (width 0.2) (layer F.Cu) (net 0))
 (segment (start 106 118.2) (end 109.8 118.2) (width 0.2) (layer F.Cu) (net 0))
 (segment (start 112.2 119) (end 115 116.2) (width 0.2) (layer F.Cu) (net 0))
 (segment (start 106 119) (end 112.2 119) (width 0.2) (layer F.Cu) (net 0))
 (segment (start 111.8 121) (end 115 124.2) (width 0.2) (layer F.Cu) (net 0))
 (segment (start 106 121) (end 111.8 121) (width 0.2) (layer F.Cu) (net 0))
 (segment (start 110.6 121.4) (end 115 125.8) (width 0.2) (layer F.Cu) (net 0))
 (segment (start 106 121.4) (end 110.6 121.4) (width 0.2) (layer F.Cu) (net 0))
 (segment (start 100.2 58.2) (end 95 53) (width 0.2) (layer F.Cu) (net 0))
 (segment (start 104 58.2) (end 100.2 58.2) (width 0.2) (layer F.Cu) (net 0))
 (segment (start 104 58.6) (end 99 58.6) (width 0.2) (layer F.Cu) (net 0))
 (segment (start 99 58.6) (end 95 54.6) (width 0.2) (layer F.Cu) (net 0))
 (segment (start 97.8 59) (end 95 56.2) (width 0.2) (layer F.Cu) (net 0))
 (segment (start 104 59) (end 97.8 59) (width 0.2) (layer F.Cu) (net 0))
 (segment (start 104 59.4) (end 96.6 59.4) (width 0.2) (layer F.Cu) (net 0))
 (segment (start 96.6 59.4) (end 95 57.8) (width 0.2) (layer F.Cu) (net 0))
 (segment (start 95.4 59.8) (end 95 59.4) (width 0.2) (layer F.Cu) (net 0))
 (segment (start 104 59.8) (end 95.4 59.8) (width 0.2) (layer F.Cu) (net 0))
 (segment (start 104 60.2) (end 95.8 60.2) (width 0.2) (layer F.Cu) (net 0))
 (segment (start 95.8 60.2) (end 95 61) (width 0.2) (layer F.Cu) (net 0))
 (segment (start 104 60.6) (end 97 60.6) (width 0.2) (layer F.Cu) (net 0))
 (segment (start 97 60.6) (end 95 62.6) (width 0.2) (layer F.Cu) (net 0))
 (segment (start 104 61) (end 98.2 61) (width 0.2) (layer F.Cu) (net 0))
 (segment (start 98.2 61) (end 95 64.2) (width 0.2) (layer F.Cu) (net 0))
 (segment (start 104 61.4) (end 99.4 61.4) (width 0.2) (layer F.Cu) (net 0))
 (segment (start 99.4 61.4) (end 95 65.8) (width 0.2) (layer F.Cu) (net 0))
 (segment (start 100.6 61.8) (end 95 67.4) (width 0.2) (layer F.Cu) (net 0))
 (segment (start 104 61.8) (end 100.6 61.8) (width 0.2) (layer F.Cu) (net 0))
 (segment (start 106 60.6) (end 113 60.6) (width 0.2) (layer F.Cu) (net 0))
 (segment (start 113 60.6) (end 115 62.6) (width 0.2) (layer F.Cu) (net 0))
 (segment (start 106 59.4) (end 113.4 59.4) (width 0.2) (layer F.Cu) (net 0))
 (segment (start 113.4 59.4) (end 115 57.8) (width 0.2) (layer F.Cu) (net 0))
 (segment (start 114.6 59.8) (end 115 59.4) (width 0.2) (layer F.Cu) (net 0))
 (segment (start 106 59.8) (end 114.6 59.8) (width 0.2) (layer F.Cu) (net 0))
 (segment (start 114.2 60.2) (end 115 61) (width 0.2) (layer F.Cu) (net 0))
 (segment (start 106 60.2) (end 114.2 60.2) (width 0.2) (layer F.Cu) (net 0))
 (segment (start 106 58.6) (end 111 58.6) (width 0.2) (layer F.Cu) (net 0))
 (segment (start 111 58.6) (end 115 54.6) (width 0.2) (layer F.Cu) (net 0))
 (segment (start 106 61.8) (end 109.4 61.8) (width 0.2) (layer F.Cu) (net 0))
 (segment (start 109.4 61.8) (end 115 67.4) (width 0.2) (layer F.Cu) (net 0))
 (segment (start 109.8 58.2) (end 115 53) (width 0.2) (layer F.Cu) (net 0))
 (segment (start 106 58.2) (end 109.8 58.2) (width 0.2) (layer F.Cu) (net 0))
 (segment (start 112.2 59) (end 115 56.2) (width 0.2) (layer F.Cu) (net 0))
 (segment (start 106 59) (end 112.2 59) (width 0.2) (layer F.Cu) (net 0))
 (segment (start 111.8 61) (end 115 64.2) (width 0.2) (layer F.Cu) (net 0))
 (segment (start 106 61) (end 111.8 61) (width 0.2) (layer F.Cu) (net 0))
 (segment (start 110.6 61.4) (end 115 65.8) (width 0.2) (layer F.Cu) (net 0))
 (segment (start 106 61.4) (end 110.6 61.4) (width 0.2) (layer F.Cu) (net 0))
 (segment (start 95 127.4) (end 95 125.8) (width 0.2) (layer F.Cu) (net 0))
 (segment (start 95 125.8) (end 95 124.2) (width 0.2) (layer F.Cu) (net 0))
 (segment (start 95 124.2) (end 95 122.6) (width 0.2) (layer F.Cu) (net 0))
 (segment (start 95 122.6) (end 95 121) (width 0.2) (layer F.Cu) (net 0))
 (segment (start 95 121) (end 95 119.4) (width 0.2) (layer F.Cu) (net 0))
 (segment (start 95 119.4) (end 95 117.8) (width 0.2) (layer F.Cu) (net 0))
 (segment (start 95 117.8) (end 95 116.2) (width 0.2) (layer F.Cu) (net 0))
 (segment (start 95 116.2) (end 95 114.6) (width 0.2) (layer F.Cu) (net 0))
 (segment (start 95 114.6) (end 95 113) (width 0.2) (layer F.Cu) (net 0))
 (segment (start 95 113) (end 95 107.4) (width 0.2) (layer F.Cu) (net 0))
 (segment (start 95 107.4) (end 95 105.8) (width 0.2) (layer F.Cu) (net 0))
 (segment (start 95 105.8) (end 95 104.2) (width 0.2) (layer F.Cu) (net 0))
 (segment (start 95 104.2) (end 95 102.6) (width 0.2) (layer F.Cu) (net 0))
 (segment (start 95 102.6) (end 95 101) (width 0.2) (layer F.Cu) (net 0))
 (segment (start 95 101) (end 95 99.4) (width 0.2) (layer F.Cu) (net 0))
 (segment (start 95 99.4) (end 95 97.8) (width 0.2) (layer F.Cu) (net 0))
 (segment (start 95 97.8) (end 95 96.2) (width 0.2) (layer F.Cu) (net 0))
 (segment (start 95 96.2) (end 95 94.6) (width 0.2) (layer F.Cu) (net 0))
 (segment (start 95 94.6) (end 95 93) (width 0.2) (layer F.Cu) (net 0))
 (segment (start 95 93) (end 95 87.4) (width 0.2) (layer F.Cu) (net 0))
 (segment (start 95 87.4) (end 95 85.8) (width 0.2) (layer F.Cu) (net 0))
 (segment (start 95 85.8) (end 95 84.2) (width 0.2) (layer F.Cu) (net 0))
 (segment (start 95 84.2) (end 95 82.6) (width 0.2) (layer F.Cu) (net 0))
 (segment (start 95 82.6) (end 95 81) (width 0.2) (layer F.Cu) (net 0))
 (segment (start 95 81) (end 95 79.4) (width 0.2) (layer F.Cu) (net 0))
 (segment (start 95 79.4) (end 95 77.8) (width 0.2) (layer F.Cu) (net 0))
 (segment (start 95 77.8) (end 95 76.2) (width 0.2) (layer F.Cu) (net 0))
 (segment (start 95 76.2) (end 95 74.6) (width 0.2) (layer F.Cu) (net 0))
 (segment (start 95 74.6) (end 95 73) (width 0.2) (layer F.Cu) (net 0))
 (segment (start 95 73) (end 95 67.4) (width 0.2) (layer F.Cu) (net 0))
 (segment (start 95 67.4) (end 95 65.8) (width 0.2) (layer F.Cu) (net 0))
 (segment (start 95 65.8) (end 95 64.2) (width 0.2) (layer F.Cu) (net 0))
 (segment (start 95 64.2) (end 95 62.6) (width 0.2) (layer F.Cu) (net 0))
 (segment (start 95 62.6) (end 95 61) (width 0.2) (layer F.Cu) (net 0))
 (segment (start 95 61) (end 95 59.4) (width 0.2) (layer F.Cu) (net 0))
 (segment (start 95 59.4) (end 95 57.8) (width 0.2) (layer F.Cu) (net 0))
 (segment (start 95 57.8) (end 95 56.2) (width 0.2) (layer F.Cu) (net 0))
 (segment (start 95 56.2) (end 95 54.6) (width 0.2) (layer F.Cu) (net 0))
 (segment (start 95 54.6) (end 95 53) (width 0.2) (layer F.Cu) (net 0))
 (segment (start 95 53) (end 95 49.6) (width 0.2) (layer F.Cu) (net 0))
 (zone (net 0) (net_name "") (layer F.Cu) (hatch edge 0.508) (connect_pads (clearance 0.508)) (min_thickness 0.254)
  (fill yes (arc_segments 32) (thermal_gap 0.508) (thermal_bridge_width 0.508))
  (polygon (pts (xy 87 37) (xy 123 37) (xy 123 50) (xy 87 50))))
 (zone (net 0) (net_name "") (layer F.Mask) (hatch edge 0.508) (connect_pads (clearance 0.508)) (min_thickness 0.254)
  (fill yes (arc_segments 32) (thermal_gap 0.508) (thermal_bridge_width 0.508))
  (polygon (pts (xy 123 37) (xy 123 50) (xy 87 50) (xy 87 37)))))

